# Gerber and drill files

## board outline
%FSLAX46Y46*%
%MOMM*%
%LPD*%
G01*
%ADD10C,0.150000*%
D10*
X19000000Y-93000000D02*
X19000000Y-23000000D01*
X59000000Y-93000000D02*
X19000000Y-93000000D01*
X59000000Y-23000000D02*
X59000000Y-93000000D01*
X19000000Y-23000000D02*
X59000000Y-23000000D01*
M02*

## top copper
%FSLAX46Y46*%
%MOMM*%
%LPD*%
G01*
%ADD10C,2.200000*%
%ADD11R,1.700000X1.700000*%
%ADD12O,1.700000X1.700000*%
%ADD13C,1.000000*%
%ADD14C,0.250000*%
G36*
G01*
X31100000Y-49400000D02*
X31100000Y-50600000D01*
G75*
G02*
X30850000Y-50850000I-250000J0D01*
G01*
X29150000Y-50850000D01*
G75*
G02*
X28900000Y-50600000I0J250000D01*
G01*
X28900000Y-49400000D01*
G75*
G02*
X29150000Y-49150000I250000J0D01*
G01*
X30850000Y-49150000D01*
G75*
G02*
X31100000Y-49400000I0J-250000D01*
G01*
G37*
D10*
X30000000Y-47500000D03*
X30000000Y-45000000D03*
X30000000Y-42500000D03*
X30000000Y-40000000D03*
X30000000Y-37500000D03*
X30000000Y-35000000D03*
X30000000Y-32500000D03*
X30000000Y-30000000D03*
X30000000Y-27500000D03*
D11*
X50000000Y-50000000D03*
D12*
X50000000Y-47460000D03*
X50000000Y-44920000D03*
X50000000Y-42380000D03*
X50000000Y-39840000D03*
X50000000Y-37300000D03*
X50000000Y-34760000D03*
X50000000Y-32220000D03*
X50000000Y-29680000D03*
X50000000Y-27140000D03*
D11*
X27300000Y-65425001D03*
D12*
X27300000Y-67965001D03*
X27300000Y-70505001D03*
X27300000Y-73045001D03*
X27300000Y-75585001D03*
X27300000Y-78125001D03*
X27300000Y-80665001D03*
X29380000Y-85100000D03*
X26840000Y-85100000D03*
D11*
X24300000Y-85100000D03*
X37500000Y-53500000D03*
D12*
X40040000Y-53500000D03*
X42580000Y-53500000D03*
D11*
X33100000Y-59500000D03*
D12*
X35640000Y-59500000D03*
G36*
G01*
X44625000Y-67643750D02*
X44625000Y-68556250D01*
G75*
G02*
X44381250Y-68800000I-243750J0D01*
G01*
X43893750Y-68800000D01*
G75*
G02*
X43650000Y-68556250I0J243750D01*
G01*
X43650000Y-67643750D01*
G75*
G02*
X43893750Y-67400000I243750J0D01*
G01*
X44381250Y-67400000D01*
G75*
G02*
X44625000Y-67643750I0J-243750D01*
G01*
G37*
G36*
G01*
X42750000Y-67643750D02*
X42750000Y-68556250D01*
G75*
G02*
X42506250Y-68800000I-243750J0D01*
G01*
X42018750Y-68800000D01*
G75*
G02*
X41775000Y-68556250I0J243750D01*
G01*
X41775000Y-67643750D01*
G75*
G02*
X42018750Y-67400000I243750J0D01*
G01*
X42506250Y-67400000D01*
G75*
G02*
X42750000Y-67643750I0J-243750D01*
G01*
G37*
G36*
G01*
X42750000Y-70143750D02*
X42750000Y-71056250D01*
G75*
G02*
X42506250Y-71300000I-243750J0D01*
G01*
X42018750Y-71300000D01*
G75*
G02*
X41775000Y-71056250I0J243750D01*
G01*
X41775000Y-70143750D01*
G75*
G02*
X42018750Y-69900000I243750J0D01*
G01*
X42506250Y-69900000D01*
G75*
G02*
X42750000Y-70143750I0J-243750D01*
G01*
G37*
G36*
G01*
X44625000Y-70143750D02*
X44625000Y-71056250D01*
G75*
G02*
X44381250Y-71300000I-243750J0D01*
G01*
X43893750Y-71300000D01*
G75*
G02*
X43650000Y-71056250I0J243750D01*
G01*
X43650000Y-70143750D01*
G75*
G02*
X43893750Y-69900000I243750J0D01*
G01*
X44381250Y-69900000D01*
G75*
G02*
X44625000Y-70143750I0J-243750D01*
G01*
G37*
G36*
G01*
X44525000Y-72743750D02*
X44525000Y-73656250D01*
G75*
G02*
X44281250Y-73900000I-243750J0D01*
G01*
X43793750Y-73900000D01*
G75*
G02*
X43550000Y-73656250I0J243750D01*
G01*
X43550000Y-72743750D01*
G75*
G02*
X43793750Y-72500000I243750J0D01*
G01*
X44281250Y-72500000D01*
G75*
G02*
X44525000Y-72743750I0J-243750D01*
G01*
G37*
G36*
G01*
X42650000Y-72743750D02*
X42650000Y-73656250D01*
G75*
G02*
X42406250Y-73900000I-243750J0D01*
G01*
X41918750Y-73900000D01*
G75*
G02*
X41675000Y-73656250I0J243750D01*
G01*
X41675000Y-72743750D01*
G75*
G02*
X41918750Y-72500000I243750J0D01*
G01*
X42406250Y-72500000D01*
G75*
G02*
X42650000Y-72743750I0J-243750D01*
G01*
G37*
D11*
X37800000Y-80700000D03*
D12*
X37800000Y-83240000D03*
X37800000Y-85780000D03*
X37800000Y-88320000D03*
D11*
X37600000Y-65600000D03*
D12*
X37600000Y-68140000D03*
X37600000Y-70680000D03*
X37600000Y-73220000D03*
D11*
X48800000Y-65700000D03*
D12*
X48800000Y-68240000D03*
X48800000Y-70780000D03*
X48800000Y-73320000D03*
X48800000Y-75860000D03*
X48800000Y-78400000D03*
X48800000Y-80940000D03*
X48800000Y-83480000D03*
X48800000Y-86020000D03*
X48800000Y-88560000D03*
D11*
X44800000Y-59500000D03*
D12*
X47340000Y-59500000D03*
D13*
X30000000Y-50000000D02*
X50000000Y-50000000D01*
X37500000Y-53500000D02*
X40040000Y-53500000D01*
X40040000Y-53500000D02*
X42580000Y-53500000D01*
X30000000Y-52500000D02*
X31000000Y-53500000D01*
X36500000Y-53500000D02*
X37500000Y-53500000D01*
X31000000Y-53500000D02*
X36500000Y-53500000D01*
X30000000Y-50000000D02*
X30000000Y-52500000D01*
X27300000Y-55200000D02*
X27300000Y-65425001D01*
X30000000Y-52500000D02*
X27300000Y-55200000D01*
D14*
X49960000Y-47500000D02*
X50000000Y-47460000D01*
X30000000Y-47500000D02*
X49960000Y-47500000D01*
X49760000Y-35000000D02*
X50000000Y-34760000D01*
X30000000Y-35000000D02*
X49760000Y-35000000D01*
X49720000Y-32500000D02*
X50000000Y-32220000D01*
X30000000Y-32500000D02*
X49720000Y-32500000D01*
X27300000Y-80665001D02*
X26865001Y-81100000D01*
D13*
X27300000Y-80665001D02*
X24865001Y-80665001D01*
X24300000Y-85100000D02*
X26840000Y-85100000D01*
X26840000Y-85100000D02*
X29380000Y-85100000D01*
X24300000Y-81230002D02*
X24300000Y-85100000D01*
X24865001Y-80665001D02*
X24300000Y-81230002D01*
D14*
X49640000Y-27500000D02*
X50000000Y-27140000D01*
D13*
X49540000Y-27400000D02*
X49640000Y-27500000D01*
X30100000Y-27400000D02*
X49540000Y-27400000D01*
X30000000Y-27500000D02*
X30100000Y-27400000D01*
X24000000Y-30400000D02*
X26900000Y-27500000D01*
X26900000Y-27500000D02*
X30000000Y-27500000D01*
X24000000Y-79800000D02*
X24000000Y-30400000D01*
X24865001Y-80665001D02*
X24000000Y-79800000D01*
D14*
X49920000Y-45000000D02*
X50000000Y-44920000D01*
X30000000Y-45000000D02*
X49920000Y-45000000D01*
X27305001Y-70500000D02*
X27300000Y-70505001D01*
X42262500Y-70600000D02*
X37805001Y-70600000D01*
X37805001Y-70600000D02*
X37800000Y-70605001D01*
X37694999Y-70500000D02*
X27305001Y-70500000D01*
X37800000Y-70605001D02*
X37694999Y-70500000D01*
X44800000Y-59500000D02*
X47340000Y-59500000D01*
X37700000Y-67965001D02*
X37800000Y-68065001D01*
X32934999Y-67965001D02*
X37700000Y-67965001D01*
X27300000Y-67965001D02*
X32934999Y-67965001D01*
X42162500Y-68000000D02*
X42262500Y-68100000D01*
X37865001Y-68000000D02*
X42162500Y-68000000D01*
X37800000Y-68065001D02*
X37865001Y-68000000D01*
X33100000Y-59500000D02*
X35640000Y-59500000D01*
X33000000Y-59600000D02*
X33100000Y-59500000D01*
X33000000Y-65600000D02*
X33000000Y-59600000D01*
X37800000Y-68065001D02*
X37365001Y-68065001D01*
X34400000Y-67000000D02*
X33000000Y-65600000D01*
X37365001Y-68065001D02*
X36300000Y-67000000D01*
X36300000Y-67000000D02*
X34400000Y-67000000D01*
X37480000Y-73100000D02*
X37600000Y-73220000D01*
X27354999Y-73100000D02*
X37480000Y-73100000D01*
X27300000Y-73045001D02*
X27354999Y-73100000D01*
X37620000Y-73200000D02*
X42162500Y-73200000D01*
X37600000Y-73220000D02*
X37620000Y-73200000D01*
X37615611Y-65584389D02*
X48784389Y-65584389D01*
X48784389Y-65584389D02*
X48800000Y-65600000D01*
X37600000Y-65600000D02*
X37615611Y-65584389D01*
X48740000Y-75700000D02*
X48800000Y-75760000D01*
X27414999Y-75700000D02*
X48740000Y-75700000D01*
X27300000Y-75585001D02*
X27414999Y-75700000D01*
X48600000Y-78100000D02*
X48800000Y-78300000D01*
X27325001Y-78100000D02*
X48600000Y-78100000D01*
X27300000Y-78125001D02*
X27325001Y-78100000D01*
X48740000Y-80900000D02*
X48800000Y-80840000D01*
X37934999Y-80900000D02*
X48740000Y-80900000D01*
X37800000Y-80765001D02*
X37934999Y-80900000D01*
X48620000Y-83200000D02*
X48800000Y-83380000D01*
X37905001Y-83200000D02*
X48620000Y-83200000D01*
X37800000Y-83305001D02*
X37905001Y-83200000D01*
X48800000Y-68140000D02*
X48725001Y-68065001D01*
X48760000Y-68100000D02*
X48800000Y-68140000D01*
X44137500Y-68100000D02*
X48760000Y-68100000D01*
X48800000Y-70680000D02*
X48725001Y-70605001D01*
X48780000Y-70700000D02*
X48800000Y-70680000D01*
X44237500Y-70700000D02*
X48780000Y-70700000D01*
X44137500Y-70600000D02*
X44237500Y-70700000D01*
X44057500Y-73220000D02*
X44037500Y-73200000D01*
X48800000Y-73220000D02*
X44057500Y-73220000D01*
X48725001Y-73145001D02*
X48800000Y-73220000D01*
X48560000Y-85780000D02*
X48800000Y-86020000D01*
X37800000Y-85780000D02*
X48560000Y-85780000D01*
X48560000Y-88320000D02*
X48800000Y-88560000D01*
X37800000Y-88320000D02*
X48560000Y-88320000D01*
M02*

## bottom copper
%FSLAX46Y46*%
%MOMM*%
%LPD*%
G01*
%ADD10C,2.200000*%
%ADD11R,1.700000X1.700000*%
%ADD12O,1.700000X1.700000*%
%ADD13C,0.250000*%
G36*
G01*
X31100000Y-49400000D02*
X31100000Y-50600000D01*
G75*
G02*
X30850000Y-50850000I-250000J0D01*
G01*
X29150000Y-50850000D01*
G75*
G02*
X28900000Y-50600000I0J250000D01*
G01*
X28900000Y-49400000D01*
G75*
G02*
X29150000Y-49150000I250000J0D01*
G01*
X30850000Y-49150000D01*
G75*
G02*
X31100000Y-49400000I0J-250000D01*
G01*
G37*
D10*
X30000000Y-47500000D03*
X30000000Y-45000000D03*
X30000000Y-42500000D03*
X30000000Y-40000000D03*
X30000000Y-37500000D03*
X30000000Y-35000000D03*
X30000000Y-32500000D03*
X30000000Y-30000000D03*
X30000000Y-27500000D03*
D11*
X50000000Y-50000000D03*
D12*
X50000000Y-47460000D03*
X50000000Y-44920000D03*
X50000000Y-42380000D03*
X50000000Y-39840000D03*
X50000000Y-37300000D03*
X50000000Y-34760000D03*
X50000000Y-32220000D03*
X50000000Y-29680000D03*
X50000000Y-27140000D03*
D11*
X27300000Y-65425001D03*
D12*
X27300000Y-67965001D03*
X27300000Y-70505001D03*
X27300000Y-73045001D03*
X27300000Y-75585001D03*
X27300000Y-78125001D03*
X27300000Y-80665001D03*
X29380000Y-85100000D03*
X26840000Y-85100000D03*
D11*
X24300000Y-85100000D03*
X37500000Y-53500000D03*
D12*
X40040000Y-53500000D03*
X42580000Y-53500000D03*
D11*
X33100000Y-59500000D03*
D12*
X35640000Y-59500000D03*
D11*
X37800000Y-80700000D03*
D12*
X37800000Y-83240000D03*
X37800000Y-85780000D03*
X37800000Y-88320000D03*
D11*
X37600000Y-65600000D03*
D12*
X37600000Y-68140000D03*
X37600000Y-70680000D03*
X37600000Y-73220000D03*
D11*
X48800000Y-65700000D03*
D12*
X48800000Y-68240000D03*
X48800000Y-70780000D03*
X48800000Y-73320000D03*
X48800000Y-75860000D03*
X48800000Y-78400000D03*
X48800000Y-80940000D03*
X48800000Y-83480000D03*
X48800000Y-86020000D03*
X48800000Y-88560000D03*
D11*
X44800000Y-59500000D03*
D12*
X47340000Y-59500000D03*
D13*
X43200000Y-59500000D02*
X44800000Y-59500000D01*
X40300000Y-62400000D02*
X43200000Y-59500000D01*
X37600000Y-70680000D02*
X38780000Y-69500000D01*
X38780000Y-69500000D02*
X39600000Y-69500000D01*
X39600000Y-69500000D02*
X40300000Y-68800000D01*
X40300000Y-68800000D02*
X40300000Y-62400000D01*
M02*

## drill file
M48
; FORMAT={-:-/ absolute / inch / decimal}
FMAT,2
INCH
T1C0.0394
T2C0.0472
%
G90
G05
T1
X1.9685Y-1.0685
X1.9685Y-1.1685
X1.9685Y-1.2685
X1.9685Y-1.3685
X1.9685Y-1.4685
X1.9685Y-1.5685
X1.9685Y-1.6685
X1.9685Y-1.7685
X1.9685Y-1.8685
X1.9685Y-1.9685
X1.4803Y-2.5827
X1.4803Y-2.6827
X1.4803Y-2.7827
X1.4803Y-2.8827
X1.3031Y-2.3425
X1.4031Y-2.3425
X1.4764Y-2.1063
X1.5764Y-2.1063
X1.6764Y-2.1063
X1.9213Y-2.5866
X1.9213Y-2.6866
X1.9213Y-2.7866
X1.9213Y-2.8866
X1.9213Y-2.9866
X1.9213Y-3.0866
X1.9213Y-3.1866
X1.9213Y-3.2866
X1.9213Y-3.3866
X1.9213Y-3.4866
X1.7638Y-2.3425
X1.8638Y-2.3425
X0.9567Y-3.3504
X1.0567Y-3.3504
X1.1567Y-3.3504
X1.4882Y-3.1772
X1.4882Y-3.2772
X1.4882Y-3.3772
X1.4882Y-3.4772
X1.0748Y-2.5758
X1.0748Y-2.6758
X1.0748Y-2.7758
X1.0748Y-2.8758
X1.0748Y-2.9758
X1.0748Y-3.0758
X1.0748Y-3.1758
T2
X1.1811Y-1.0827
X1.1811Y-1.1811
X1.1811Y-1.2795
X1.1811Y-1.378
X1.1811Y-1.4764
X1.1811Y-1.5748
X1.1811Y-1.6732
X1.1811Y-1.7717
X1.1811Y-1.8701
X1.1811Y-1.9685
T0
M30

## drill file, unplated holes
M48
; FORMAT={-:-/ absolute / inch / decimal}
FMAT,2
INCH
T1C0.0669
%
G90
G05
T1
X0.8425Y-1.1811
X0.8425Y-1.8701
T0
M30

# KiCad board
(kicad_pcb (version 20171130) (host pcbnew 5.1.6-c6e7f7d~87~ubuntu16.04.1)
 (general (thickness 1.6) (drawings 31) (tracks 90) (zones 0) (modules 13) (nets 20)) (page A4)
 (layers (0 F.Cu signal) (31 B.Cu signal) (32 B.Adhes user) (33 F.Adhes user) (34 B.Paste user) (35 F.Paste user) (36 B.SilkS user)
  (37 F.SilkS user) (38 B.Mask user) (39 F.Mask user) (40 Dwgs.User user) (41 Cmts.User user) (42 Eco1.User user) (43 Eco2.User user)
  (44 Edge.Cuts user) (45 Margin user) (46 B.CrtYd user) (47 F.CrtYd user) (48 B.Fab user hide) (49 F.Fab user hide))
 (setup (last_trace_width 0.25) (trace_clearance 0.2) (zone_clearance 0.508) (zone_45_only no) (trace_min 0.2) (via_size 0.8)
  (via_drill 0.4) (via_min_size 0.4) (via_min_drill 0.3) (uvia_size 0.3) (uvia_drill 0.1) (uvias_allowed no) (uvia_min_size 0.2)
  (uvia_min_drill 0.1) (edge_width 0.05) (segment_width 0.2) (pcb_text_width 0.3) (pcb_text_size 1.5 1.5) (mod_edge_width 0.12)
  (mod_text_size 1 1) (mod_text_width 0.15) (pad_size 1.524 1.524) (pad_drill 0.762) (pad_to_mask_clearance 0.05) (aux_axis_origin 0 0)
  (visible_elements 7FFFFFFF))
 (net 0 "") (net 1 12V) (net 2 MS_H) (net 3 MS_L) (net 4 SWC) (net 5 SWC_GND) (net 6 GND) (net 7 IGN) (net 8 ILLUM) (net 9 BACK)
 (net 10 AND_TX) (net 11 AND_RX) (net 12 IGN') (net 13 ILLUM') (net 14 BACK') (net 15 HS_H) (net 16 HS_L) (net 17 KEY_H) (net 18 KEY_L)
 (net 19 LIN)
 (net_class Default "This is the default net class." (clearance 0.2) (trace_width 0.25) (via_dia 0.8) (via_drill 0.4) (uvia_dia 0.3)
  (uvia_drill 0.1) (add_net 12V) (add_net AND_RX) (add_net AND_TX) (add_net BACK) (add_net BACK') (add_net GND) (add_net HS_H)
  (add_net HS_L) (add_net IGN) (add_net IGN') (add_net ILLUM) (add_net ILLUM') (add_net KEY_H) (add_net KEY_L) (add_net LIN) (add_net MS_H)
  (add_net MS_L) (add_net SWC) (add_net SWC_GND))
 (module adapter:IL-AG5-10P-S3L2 (layer F.Cu) (at 30 50 180)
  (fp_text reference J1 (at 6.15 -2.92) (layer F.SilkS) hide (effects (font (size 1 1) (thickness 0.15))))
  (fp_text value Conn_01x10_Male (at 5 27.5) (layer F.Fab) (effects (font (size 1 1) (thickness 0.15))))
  (pad 1 thru_hole roundrect (at 0 0 180) (size 2.2 1.7) (drill 1.2) (layers *.Cu *.Mask) (roundrect_rratio 0.147059) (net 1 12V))
  (pad 2 thru_hole circle (at 0 2.5 180) (size 2.2 2.2) (drill 1.2) (layers *.Cu *.Mask) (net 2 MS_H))
  (pad 3 thru_hole circle (at 0 5 180) (size 2.2 2.2) (drill 1.2) (layers *.Cu *.Mask) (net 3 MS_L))
  (pad 4 thru_hole circle (at 0 7.5 180) (size 2.2 2.2) (drill 1.2) (layers *.Cu *.Mask))
  (pad 5 thru_hole circle (at 0 10 180) (size 2.2 2.2) (drill 1.2) (layers *.Cu *.Mask))
  (pad 6 thru_hole circle (at 0 12.5 180) (size 2.2 2.2) (drill 1.2) (layers *.Cu *.Mask))
  (pad 7 thru_hole circle (at 0 15 180) (size 2.2 2.2) (drill 1.2) (layers *.Cu *.Mask) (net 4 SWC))
  (pad 8 thru_hole circle (at 0 17.5 180) (size 2.2 2.2) (drill 1.2) (layers *.Cu *.Mask) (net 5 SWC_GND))
  (pad "" np_thru_hole circle (at 8.6 2.5 180) (size 1.7 1.7) (drill 1.7) (layers *.Cu *.Mask))
  (pad "" np_thru_hole circle (at 8.6 20 180) (size 1.7 1.7) (drill 1.7) (layers *.Cu *.Mask))
  (pad 9 thru_hole circle (at 0 20 180) (size 2.2 2.2) (drill 1.2) (layers *.Cu *.Mask))
  (pad 10 thru_hole circle (at 0 22.5 180) (size 2.2 2.2) (drill 1.2) (layers *.Cu *.Mask) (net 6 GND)))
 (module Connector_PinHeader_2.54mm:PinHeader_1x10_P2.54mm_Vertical (layer F.Cu) (at 50 50 180)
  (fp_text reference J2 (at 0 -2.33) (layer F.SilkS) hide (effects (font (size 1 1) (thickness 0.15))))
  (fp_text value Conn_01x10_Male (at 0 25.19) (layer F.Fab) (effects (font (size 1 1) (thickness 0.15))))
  (pad 1 thru_hole rect (at 0 0 180) (size 1.7 1.7) (drill 1) (layers *.Cu *.Mask) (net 1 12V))
  (pad 2 thru_hole oval (at 0 2.54 180) (size 1.7 1.7) (drill 1) (layers *.Cu *.Mask) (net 2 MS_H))
  (pad 3 thru_hole oval (at 0 5.08 180) (size 1.7 1.7) (drill 1) (layers *.Cu *.Mask) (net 3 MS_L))
  (pad 4 thru_hole oval (at 0 7.62 180) (size 1.7 1.7) (drill 1) (layers *.Cu *.Mask))
  (pad 5 thru_hole oval (at 0 10.16 180) (size 1.7 1.7) (drill 1) (layers *.Cu *.Mask))
  (pad 6 thru_hole oval (at 0 12.7 180) (size 1.7 1.7) (drill 1) (layers *.Cu *.Mask))
  (pad 7 thru_hole oval (at 0 15.24 180) (size 1.7 1.7) (drill 1) (layers *.Cu *.Mask) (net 4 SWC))
  (pad 8 thru_hole oval (at 0 17.78 180) (size 1.7 1.7) (drill 1) (layers *.Cu *.Mask) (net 5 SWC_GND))
  (pad 9 thru_hole oval (at 0 20.32 180) (size 1.7 1.7) (drill 1) (layers *.Cu *.Mask))
  (pad 10 thru_hole oval (at 0 22.86 180) (size 1.7 1.7) (drill 1) (layers *.Cu *.Mask) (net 6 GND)))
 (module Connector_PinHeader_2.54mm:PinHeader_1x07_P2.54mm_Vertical (layer F.Cu) (at 27.3 65.425001)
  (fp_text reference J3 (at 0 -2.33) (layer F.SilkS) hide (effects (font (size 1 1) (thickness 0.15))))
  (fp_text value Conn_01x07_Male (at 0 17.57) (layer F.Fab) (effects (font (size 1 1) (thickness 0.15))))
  (pad 1 thru_hole rect (at 0 0) (size 1.7 1.7) (drill 1) (layers *.Cu *.Mask) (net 1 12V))
  (pad 2 thru_hole oval (at 0 2.54) (size 1.7 1.7) (drill 1) (layers *.Cu *.Mask) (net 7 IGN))
  (pad 3 thru_hole oval (at 0 5.08) (size 1.7 1.7) (drill 1) (layers *.Cu *.Mask) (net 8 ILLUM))
  (pad 4 thru_hole oval (at 0 7.62) (size 1.7 1.7) (drill 1) (layers *.Cu *.Mask) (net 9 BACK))
  (pad 5 thru_hole oval (at 0 10.16) (size 1.7 1.7) (drill 1) (layers *.Cu *.Mask) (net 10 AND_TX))
  (pad 6 thru_hole oval (at 0 12.7) (size 1.7 1.7) (drill 1) (layers *.Cu *.Mask) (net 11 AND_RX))
  (pad 7 thru_hole oval (at 0 15.24) (size 1.7 1.7) (drill 1) (layers *.Cu *.Mask) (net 6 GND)))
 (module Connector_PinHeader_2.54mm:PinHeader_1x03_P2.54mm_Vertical (layer F.Cu) (at 24.3 85.1 90)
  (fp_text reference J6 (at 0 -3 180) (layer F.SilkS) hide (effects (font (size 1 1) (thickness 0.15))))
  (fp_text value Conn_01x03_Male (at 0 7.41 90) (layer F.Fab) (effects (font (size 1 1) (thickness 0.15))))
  (pad 3 thru_hole oval (at 0 5.08 90) (size 1.7 1.7) (drill 1) (layers *.Cu *.Mask) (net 6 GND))
  (pad 2 thru_hole oval (at 0 2.54 90) (size 1.7 1.7) (drill 1) (layers *.Cu *.Mask) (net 6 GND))
  (pad 1 thru_hole rect (at 0 0 90) (size 1.7 1.7) (drill 1) (layers *.Cu *.Mask) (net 6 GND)))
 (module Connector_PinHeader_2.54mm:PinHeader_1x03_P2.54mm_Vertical (layer F.Cu) (at 37.5 53.5 90)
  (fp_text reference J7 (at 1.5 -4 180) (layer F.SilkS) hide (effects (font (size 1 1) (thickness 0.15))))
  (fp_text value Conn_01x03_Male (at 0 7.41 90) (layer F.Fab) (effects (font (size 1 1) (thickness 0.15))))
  (pad 1 thru_hole rect (at 0 0 90) (size 1.7 1.7) (drill 1) (layers *.Cu *.Mask) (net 1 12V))
  (pad 2 thru_hole oval (at 0 2.54 90) (size 1.7 1.7) (drill 1) (layers *.Cu *.Mask) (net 1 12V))
  (pad 3 thru_hole oval (at 0 5.08 90) (size 1.7 1.7) (drill 1) (layers *.Cu *.Mask) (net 1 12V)))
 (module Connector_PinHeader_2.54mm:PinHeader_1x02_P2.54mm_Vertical (layer F.Cu) (at 33.1 59.5 90)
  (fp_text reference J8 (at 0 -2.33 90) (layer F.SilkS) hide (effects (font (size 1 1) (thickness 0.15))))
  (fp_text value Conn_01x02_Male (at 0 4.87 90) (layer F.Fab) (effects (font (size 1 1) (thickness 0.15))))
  (pad 1 thru_hole rect (at 0 0 90) (size 1.7 1.7) (drill 1) (layers *.Cu *.Mask) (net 7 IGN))
  (pad 2 thru_hole oval (at 0 2.54 90) (size 1.7 1.7) (drill 1) (layers *.Cu *.Mask) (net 7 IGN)))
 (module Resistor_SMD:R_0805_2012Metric (layer F.Cu) (at 43.2 68.1 180)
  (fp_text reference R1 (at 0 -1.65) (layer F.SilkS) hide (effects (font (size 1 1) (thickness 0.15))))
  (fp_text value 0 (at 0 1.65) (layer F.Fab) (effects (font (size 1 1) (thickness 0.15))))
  (pad 1 smd roundrect (at -0.9375 0 180) (size 0.975 1.4) (layers F.Cu F.Paste F.Mask) (roundrect_rratio 0.25) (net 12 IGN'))
  (pad 2 smd roundrect (at 0.9375 0 180) (size 0.975 1.4) (layers F.Cu F.Paste F.Mask) (roundrect_rratio 0.25) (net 7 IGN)))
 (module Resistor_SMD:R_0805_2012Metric (layer F.Cu) (at 43.2 70.6 180)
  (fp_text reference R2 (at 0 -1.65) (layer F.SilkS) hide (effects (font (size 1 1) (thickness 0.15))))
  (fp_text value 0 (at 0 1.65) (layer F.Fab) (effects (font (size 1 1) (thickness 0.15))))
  (pad 2 smd roundrect (at 0.9375 0 180) (size 0.975 1.4) (layers F.Cu F.Paste F.Mask) (roundrect_rratio 0.25) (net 8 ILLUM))
  (pad 1 smd roundrect (at -0.9375 0 180) (size 0.975 1.4) (layers F.Cu F.Paste F.Mask) (roundrect_rratio 0.25) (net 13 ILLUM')))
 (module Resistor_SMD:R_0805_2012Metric (layer F.Cu) (at 43.1 73.2 180)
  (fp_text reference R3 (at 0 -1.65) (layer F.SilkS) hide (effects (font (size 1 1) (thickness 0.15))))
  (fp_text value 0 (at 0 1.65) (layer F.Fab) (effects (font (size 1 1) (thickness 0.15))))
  (pad 1 smd roundrect (at -0.9375 0 180) (size 0.975 1.4) (layers F.Cu F.Paste F.Mask) (roundrect_rratio 0.25) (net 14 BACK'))
  (pad 2 smd roundrect (at 0.9375 0 180) (size 0.975 1.4) (layers F.Cu F.Paste F.Mask) (roundrect_rratio 0.25) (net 9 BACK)))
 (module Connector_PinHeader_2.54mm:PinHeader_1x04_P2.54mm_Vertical (layer F.Cu) (at 37.8 80.7)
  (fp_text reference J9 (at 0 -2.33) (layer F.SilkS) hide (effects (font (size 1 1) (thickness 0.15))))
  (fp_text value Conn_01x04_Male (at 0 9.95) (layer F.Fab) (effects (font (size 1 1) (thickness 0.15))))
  (pad 1 thru_hole rect (at 0 0) (size 1.7 1.7) (drill 1) (layers *.Cu *.Mask) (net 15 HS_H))
  (pad 2 thru_hole oval (at 0 2.54) (size 1.7 1.7) (drill 1) (layers *.Cu *.Mask) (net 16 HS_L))
  (pad 3 thru_hole oval (at 0 5.08) (size 1.7 1.7) (drill 1) (layers *.Cu *.Mask) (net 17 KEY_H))
  (pad 4 thru_hole oval (at 0 7.62) (size 1.7 1.7) (drill 1) (layers *.Cu *.Mask) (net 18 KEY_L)))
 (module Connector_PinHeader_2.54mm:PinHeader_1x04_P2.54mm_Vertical (layer F.Cu) (at 37.6 65.6)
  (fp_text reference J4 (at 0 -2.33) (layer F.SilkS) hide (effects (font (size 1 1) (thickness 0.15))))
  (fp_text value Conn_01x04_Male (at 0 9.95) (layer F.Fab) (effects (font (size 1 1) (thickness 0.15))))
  (pad 1 thru_hole rect (at 0 0) (size 1.7 1.7) (drill 1) (layers *.Cu *.Mask) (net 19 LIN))
  (pad 2 thru_hole oval (at 0 2.54) (size 1.7 1.7) (drill 1) (layers *.Cu *.Mask) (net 7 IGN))
  (pad 3 thru_hole oval (at 0 5.08) (size 1.7 1.7) (drill 1) (layers *.Cu *.Mask) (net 8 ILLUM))
  (pad 4 thru_hole oval (at 0 7.62) (size 1.7 1.7) (drill 1) (layers *.Cu *.Mask) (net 9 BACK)))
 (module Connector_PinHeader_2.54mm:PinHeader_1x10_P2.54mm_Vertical (layer F.Cu) (at 48.8 65.7)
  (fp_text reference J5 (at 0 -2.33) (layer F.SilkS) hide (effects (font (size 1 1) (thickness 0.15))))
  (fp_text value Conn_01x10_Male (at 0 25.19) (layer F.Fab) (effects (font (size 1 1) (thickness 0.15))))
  (pad 1 thru_hole rect (at 0 0) (size 1.7 1.7) (drill 1) (layers *.Cu *.Mask) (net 19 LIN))
  (pad 2 thru_hole oval (at 0 2.54) (size 1.7 1.7) (drill 1) (layers *.Cu *.Mask) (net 12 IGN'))
  (pad 3 thru_hole oval (at 0 5.08) (size 1.7 1.7) (drill 1) (layers *.Cu *.Mask) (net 13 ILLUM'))
  (pad 4 thru_hole oval (at 0 7.62) (size 1.7 1.7) (drill 1) (layers *.Cu *.Mask) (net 14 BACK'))
  (pad 5 thru_hole oval (at 0 10.16) (size 1.7 1.7) (drill 1) (layers *.Cu *.Mask) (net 10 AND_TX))
  (pad 6 thru_hole oval (at 0 12.7) (size 1.7 1.7) (drill 1) (layers *.Cu *.Mask) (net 11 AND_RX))
  (pad 7 thru_hole oval (at 0 15.24) (size 1.7 1.7) (drill 1) (layers *.Cu *.Mask) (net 15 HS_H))
  (pad 8 thru_hole oval (at 0 17.78) (size 1.7 1.7) (drill 1) (layers *.Cu *.Mask) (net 16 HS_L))
  (pad 9 thru_hole oval (at 0 20.32) (size 1.7 1.7) (drill 1) (layers *.Cu *.Mask) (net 17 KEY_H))
  (pad 10 thru_hole oval (at 0 22.86) (size 1.7 1.7) (drill 1) (layers *.Cu *.Mask) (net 18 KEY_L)))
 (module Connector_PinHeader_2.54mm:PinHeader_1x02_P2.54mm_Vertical (layer F.Cu) (at 44.8 59.5 90)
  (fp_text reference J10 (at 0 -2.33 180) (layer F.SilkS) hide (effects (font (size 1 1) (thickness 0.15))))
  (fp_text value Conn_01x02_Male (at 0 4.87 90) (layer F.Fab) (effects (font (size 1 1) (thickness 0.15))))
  (pad 1 thru_hole rect (at 0 0 90) (size 1.7 1.7) (drill 1) (layers *.Cu *.Mask) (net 8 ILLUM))
  (pad 2 thru_hole oval (at 0 2.54 90) (size 1.7 1.7) (drill 1) (layers *.Cu *.Mask) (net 8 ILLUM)))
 (gr_line (start 19 93) (end 19 23) (layer Edge.Cuts) (width 0.15))
 (gr_line (start 59 93) (end 19 93) (layer Edge.Cuts) (width 0.15))
 (gr_line (start 59 23) (end 59 93) (layer Edge.Cuts) (width 0.15))
 (gr_line (start 19 23) (end 59 23) (layer Edge.Cuts) (width 0.15))
 (segment (start 30 50) (end 50 50) (width 1) (layer F.Cu) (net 1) (status 30))
 (segment (start 37.5 53.5) (end 40.04 53.5) (width 1) (layer F.Cu) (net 1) (status 30))
 (segment (start 40.04 53.5) (end 42.58 53.5) (width 1) (layer F.Cu) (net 1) (status 30))
 (segment (start 30 52.5) (end 31 53.5) (width 1) (layer F.Cu) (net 1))
 (segment (start 36.5 53.5) (end 37.5 53.5) (width 1) (layer F.Cu) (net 1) (status 20))
 (segment (start 31 53.5) (end 36.5 53.5) (width 1) (layer F.Cu) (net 1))
 (segment (start 30 50) (end 30 52.5) (width 1) (layer F.Cu) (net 1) (status 10))
 (segment (start 27.3 55.2) (end 27.3 65.425001) (width 1) (layer F.Cu) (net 1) (status 20))
 (segment (start 30 52.5) (end 27.3 55.2) (width 1) (layer F.Cu) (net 1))
 (segment (start 49.96 47.5) (end 50 47.46) (width 0.25) (layer F.Cu) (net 2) (status 30))
 (segment (start 30 47.5) (end 49.96 47.5) (width 0.25) (layer F.Cu) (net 2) (status 30))
 (segment (start 49.76 35) (end 50 34.76) (width 0.25) (layer F.Cu) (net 4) (status 30))
 (segment (start 30 35) (end 49.76 35) (width 0.25) (layer F.Cu) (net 4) (status 30))
 (segment (start 49.72 32.5) (end 50 32.22) (width 0.25) (layer F.Cu) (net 5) (status 30))
 (segment (start 30 32.5) (end 49.72 32.5) (width 0.25) (layer F.Cu) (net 5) (status 30))
 (segment (start 27.3 80.665001) (end 26.865001 81.1) (width 0.25) (layer F.Cu) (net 6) (status 30))
 (segment (start 27.3 80.665001) (end 24.865001 80.665001) (width 1) (layer F.Cu) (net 6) (status 10))
 (segment (start 24.3 85.1) (end 26.84 85.1) (width 1) (layer F.Cu) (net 6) (status 30))
 (segment (start 26.84 85.1) (end 29.38 85.1) (width 1) (layer F.Cu) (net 6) (status 30))
 (segment (start 24.3 81.230002) (end 24.3 85.1) (width 1) (layer F.Cu) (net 6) (status 20))
 (segment (start 24.865001 80.665001) (end 24.3 81.230002) (width 1) (layer F.Cu) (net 6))
 (segment (start 49.64 27.5) (end 50 27.14) (width 0.25) (layer F.Cu) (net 6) (status 30))
 (segment (start 49.54 27.4) (end 49.64 27.5) (width 1) (layer F.Cu) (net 6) (status 30))
 (segment (start 30.1 27.4) (end 49.54 27.4) (width 1) (layer F.Cu) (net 6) (status 30))
 (segment (start 30 27.5) (end 30.1 27.4) (width 1) (layer F.Cu) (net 6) (status 30))
 (segment (start 24 30.4) (end 26.9 27.5) (width 1) (layer F.Cu) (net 6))
 (segment (start 26.9 27.5) (end 30 27.5) (width 1) (layer F.Cu) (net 6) (status 20))
 (segment (start 24 79.8) (end 24 30.4) (width 1) (layer F.Cu) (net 6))
 (segment (start 24.865001 80.665001) (end 24 79.8) (width 1) (layer F.Cu) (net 6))
 (segment (start 49.92 45) (end 50 44.92) (width 0.25) (layer F.Cu) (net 3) (status 30))
 (segment (start 30 45) (end 49.92 45) (width 0.25) (layer F.Cu) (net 3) (status 30))
 (segment (start 27.305001 70.5) (end 27.3 70.505001) (width 0.25) (layer F.Cu) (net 8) (status 30))
 (segment (start 42.2625 70.6) (end 37.805001 70.6) (width 0.25) (layer F.Cu) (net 8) (status 30))
 (segment (start 37.805001 70.6) (end 37.8 70.605001) (width 0.25) (layer F.Cu) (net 8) (status 30))
 (segment (start 37.694999 70.5) (end 27.305001 70.5) (width 0.25) (layer F.Cu) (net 8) (status 30))
 (segment (start 37.8 70.605001) (end 37.694999 70.5) (width 0.25) (layer F.Cu) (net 8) (status 30))
 (segment (start 44.8 59.5) (end 47.34 59.5) (width 0.25) (layer F.Cu) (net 8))
 (segment (start 43.2 59.5) (end 44.8 59.5) (width 0.25) (layer B.Cu) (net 8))
 (segment (start 40.3 62.4) (end 43.2 59.5) (width 0.25) (layer B.Cu) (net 8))
 (segment (start 37.6 70.68) (end 38.78 69.5) (width 0.25) (layer B.Cu) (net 8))
 (segment (start 38.78 69.5) (end 39.6 69.5) (width 0.25) (layer B.Cu) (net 8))
 (segment (start 39.6 69.5) (end 40.3 68.8) (width 0.25) (layer B.Cu) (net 8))
 (segment (start 40.3 68.8) (end 40.3 62.4) (width 0.25) (layer B.Cu) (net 8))
 (segment (start 37.7 67.965001) (end 37.8 68.065001) (width 0.25) (layer F.Cu) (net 7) (status 30))
 (segment (start 32.934999 67.965001) (end 37.7 67.965001) (width 0.25) (layer F.Cu) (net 7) (status 20))
 (segment (start 27.3 67.965001) (end 32.934999 67.965001) (width 0.25) (layer F.Cu) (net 7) (status 10))
 (segment (start 42.1625 68) (end 42.2625 68.1) (width 0.25) (layer F.Cu) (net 7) (status 30))
 (segment (start 37.865001 68) (end 42.1625 68) (width 0.25) (layer F.Cu) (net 7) (status 30))
 (segment (start 37.8 68.065001) (end 37.865001 68) (width 0.25) (layer F.Cu) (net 7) (status 30))
 (segment (start 33.1 59.5) (end 35.64 59.5) (width 0.25) (layer F.Cu) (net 7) (status 30))
 (segment (start 33 59.6) (end 33.1 59.5) (width 0.25) (layer F.Cu) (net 7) (status 30))
 (segment (start 33 65.6) (end 33 59.6) (width 0.25) (layer F.Cu) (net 7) (status 20))
 (segment (start 37.8 68.065001) (end 37.365001 68.065001) (width 0.25) (layer F.Cu) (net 7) (status 30))
 (segment (start 34.4 67) (end 33 65.6) (width 0.25) (layer F.Cu) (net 7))
 (segment (start 37.365001 68.065001) (end 36.3 67) (width 0.25) (layer F.Cu) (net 7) (status 10))
 (segment (start 36.3 67) (end 34.4 67) (width 0.25) (layer F.Cu) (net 7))
 (segment (start 37.48 73.1) (end 37.6 73.22) (width 0.25) (layer F.Cu) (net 9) (status 30))
 (segment (start 27.354999 73.1) (end 37.48 73.1) (width 0.25) (layer F.Cu) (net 9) (status 30))
 (segment (start 27.3 73.045001) (end 27.354999 73.1) (width 0.25) (layer F.Cu) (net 9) (status 30))
 (segment (start 37.62 73.2) (end 42.1625 73.2) (width 0.25) (layer F.Cu) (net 9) (status 30))
 (segment (start 37.6 73.22) (end 37.62 73.2) (width 0.25) (layer F.Cu) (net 9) (status 30))
 (segment (start 37.615611 65.584389) (end 48.784389 65.584389) (width 0.25) (layer F.Cu) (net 19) (status 30))
 (segment (start 48.784389 65.584389) (end 48.8 65.6) (width 0.25) (layer F.Cu) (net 19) (status 30))
 (segment (start 37.6 65.6) (end 37.615611 65.584389) (width 0.25) (layer F.Cu) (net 19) (status 30))
 (segment (start 48.74 75.7) (end 48.8 75.76) (width 0.25) (layer F.Cu) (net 10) (status 30))
 (segment (start 27.414999 75.7) (end 48.74 75.7) (width 0.25) (layer F.Cu) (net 10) (status 30))
 (segment (start 27.3 75.585001) (end 27.414999 75.7) (width 0.25) (layer F.Cu) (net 10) (status 30))
 (segment (start 48.6 78.1) (end 48.8 78.3) (width 0.25) (layer F.Cu) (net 11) (status 30))
 (segment (start 27.325001 78.1) (end 48.6 78.1) (width 0.25) (layer F.Cu) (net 11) (status 30))
 (segment (start 27.3 78.125001) (end 27.325001 78.1) (width 0.25) (layer F.Cu) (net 11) (status 30))
 (segment (start 48.74 80.9) (end 48.8 80.84) (width 0.25) (layer F.Cu) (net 15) (status 30))
 (segment (start 37.934999 80.9) (end 48.74 80.9) (width 0.25) (layer F.Cu) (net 15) (status 30))
 (segment (start 37.8 80.765001) (end 37.934999 80.9) (width 0.25) (layer F.Cu) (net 15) (status 30))
 (segment (start 48.62 83.2) (end 48.8 83.38) (width 0.25) (layer F.Cu) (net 16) (status 30))
 (segment (start 37.905001 83.2) (end 48.62 83.2) (width 0.25) (layer F.Cu) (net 16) (status 30))
 (segment (start 37.8 83.305001) (end 37.905001 83.2) (width 0.25) (layer F.Cu) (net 16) (status 30))
 (segment (start 48.8 68.14) (end 48.725001 68.065001) (width 0.25) (layer F.Cu) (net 12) (status 30))
 (segment (start 48.76 68.1) (end 48.8 68.14) (width 0.25) (layer F.Cu) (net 12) (status 30))
 (segment (start 44.1375 68.1) (end 48.76 68.1) (width 0.25) (layer F.Cu) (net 12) (status 30))
 (segment (start 48.8 70.68) (end 48.725001 70.605001) (width 0.25) (layer F.Cu) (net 13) (status 30))
 (segment (start 48.78 70.7) (end 48.8 70.68) (width 0.25) (layer F.Cu) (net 13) (status 30))
 (segment (start 44.2375 70.7) (end 48.78 70.7) (width 0.25) (layer F.Cu) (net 13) (status 30))
 (segment (start 44.1375 70.6) (end 44.2375 70.7) (width 0.25) (layer F.Cu) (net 13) (status 30))
 (segment (start 44.0575 73.22) (end 44.0375 73.2) (width 0.25) (layer F.Cu) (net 14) (status 30))
 (segment (start 48.8 73.22) (end 44.0575 73.22) (width 0.25) (layer F.Cu) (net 14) (status 30))
 (segment (start 48.725001 73.145001) (end 48.8 73.22) (width 0.25) (layer F.Cu) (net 14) (status 30))
 (segment (start 48.56 85.78) (end 48.8 86.02) (width 0.25) (layer F.Cu) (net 17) (status 30))
 (segment (start 37.8 85.78) (end 48.56 85.78) (width 0.25) (layer F.Cu) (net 17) (status 30))
 (segment (start 48.56 88.32) (end 48.8 88.56) (width 0.25) (layer F.Cu) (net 18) (status 30))
 (segment (start 37.8 88.32) (end 48.56 88.32) (width 0.25) (layer F.Cu) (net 18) (status 30)))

